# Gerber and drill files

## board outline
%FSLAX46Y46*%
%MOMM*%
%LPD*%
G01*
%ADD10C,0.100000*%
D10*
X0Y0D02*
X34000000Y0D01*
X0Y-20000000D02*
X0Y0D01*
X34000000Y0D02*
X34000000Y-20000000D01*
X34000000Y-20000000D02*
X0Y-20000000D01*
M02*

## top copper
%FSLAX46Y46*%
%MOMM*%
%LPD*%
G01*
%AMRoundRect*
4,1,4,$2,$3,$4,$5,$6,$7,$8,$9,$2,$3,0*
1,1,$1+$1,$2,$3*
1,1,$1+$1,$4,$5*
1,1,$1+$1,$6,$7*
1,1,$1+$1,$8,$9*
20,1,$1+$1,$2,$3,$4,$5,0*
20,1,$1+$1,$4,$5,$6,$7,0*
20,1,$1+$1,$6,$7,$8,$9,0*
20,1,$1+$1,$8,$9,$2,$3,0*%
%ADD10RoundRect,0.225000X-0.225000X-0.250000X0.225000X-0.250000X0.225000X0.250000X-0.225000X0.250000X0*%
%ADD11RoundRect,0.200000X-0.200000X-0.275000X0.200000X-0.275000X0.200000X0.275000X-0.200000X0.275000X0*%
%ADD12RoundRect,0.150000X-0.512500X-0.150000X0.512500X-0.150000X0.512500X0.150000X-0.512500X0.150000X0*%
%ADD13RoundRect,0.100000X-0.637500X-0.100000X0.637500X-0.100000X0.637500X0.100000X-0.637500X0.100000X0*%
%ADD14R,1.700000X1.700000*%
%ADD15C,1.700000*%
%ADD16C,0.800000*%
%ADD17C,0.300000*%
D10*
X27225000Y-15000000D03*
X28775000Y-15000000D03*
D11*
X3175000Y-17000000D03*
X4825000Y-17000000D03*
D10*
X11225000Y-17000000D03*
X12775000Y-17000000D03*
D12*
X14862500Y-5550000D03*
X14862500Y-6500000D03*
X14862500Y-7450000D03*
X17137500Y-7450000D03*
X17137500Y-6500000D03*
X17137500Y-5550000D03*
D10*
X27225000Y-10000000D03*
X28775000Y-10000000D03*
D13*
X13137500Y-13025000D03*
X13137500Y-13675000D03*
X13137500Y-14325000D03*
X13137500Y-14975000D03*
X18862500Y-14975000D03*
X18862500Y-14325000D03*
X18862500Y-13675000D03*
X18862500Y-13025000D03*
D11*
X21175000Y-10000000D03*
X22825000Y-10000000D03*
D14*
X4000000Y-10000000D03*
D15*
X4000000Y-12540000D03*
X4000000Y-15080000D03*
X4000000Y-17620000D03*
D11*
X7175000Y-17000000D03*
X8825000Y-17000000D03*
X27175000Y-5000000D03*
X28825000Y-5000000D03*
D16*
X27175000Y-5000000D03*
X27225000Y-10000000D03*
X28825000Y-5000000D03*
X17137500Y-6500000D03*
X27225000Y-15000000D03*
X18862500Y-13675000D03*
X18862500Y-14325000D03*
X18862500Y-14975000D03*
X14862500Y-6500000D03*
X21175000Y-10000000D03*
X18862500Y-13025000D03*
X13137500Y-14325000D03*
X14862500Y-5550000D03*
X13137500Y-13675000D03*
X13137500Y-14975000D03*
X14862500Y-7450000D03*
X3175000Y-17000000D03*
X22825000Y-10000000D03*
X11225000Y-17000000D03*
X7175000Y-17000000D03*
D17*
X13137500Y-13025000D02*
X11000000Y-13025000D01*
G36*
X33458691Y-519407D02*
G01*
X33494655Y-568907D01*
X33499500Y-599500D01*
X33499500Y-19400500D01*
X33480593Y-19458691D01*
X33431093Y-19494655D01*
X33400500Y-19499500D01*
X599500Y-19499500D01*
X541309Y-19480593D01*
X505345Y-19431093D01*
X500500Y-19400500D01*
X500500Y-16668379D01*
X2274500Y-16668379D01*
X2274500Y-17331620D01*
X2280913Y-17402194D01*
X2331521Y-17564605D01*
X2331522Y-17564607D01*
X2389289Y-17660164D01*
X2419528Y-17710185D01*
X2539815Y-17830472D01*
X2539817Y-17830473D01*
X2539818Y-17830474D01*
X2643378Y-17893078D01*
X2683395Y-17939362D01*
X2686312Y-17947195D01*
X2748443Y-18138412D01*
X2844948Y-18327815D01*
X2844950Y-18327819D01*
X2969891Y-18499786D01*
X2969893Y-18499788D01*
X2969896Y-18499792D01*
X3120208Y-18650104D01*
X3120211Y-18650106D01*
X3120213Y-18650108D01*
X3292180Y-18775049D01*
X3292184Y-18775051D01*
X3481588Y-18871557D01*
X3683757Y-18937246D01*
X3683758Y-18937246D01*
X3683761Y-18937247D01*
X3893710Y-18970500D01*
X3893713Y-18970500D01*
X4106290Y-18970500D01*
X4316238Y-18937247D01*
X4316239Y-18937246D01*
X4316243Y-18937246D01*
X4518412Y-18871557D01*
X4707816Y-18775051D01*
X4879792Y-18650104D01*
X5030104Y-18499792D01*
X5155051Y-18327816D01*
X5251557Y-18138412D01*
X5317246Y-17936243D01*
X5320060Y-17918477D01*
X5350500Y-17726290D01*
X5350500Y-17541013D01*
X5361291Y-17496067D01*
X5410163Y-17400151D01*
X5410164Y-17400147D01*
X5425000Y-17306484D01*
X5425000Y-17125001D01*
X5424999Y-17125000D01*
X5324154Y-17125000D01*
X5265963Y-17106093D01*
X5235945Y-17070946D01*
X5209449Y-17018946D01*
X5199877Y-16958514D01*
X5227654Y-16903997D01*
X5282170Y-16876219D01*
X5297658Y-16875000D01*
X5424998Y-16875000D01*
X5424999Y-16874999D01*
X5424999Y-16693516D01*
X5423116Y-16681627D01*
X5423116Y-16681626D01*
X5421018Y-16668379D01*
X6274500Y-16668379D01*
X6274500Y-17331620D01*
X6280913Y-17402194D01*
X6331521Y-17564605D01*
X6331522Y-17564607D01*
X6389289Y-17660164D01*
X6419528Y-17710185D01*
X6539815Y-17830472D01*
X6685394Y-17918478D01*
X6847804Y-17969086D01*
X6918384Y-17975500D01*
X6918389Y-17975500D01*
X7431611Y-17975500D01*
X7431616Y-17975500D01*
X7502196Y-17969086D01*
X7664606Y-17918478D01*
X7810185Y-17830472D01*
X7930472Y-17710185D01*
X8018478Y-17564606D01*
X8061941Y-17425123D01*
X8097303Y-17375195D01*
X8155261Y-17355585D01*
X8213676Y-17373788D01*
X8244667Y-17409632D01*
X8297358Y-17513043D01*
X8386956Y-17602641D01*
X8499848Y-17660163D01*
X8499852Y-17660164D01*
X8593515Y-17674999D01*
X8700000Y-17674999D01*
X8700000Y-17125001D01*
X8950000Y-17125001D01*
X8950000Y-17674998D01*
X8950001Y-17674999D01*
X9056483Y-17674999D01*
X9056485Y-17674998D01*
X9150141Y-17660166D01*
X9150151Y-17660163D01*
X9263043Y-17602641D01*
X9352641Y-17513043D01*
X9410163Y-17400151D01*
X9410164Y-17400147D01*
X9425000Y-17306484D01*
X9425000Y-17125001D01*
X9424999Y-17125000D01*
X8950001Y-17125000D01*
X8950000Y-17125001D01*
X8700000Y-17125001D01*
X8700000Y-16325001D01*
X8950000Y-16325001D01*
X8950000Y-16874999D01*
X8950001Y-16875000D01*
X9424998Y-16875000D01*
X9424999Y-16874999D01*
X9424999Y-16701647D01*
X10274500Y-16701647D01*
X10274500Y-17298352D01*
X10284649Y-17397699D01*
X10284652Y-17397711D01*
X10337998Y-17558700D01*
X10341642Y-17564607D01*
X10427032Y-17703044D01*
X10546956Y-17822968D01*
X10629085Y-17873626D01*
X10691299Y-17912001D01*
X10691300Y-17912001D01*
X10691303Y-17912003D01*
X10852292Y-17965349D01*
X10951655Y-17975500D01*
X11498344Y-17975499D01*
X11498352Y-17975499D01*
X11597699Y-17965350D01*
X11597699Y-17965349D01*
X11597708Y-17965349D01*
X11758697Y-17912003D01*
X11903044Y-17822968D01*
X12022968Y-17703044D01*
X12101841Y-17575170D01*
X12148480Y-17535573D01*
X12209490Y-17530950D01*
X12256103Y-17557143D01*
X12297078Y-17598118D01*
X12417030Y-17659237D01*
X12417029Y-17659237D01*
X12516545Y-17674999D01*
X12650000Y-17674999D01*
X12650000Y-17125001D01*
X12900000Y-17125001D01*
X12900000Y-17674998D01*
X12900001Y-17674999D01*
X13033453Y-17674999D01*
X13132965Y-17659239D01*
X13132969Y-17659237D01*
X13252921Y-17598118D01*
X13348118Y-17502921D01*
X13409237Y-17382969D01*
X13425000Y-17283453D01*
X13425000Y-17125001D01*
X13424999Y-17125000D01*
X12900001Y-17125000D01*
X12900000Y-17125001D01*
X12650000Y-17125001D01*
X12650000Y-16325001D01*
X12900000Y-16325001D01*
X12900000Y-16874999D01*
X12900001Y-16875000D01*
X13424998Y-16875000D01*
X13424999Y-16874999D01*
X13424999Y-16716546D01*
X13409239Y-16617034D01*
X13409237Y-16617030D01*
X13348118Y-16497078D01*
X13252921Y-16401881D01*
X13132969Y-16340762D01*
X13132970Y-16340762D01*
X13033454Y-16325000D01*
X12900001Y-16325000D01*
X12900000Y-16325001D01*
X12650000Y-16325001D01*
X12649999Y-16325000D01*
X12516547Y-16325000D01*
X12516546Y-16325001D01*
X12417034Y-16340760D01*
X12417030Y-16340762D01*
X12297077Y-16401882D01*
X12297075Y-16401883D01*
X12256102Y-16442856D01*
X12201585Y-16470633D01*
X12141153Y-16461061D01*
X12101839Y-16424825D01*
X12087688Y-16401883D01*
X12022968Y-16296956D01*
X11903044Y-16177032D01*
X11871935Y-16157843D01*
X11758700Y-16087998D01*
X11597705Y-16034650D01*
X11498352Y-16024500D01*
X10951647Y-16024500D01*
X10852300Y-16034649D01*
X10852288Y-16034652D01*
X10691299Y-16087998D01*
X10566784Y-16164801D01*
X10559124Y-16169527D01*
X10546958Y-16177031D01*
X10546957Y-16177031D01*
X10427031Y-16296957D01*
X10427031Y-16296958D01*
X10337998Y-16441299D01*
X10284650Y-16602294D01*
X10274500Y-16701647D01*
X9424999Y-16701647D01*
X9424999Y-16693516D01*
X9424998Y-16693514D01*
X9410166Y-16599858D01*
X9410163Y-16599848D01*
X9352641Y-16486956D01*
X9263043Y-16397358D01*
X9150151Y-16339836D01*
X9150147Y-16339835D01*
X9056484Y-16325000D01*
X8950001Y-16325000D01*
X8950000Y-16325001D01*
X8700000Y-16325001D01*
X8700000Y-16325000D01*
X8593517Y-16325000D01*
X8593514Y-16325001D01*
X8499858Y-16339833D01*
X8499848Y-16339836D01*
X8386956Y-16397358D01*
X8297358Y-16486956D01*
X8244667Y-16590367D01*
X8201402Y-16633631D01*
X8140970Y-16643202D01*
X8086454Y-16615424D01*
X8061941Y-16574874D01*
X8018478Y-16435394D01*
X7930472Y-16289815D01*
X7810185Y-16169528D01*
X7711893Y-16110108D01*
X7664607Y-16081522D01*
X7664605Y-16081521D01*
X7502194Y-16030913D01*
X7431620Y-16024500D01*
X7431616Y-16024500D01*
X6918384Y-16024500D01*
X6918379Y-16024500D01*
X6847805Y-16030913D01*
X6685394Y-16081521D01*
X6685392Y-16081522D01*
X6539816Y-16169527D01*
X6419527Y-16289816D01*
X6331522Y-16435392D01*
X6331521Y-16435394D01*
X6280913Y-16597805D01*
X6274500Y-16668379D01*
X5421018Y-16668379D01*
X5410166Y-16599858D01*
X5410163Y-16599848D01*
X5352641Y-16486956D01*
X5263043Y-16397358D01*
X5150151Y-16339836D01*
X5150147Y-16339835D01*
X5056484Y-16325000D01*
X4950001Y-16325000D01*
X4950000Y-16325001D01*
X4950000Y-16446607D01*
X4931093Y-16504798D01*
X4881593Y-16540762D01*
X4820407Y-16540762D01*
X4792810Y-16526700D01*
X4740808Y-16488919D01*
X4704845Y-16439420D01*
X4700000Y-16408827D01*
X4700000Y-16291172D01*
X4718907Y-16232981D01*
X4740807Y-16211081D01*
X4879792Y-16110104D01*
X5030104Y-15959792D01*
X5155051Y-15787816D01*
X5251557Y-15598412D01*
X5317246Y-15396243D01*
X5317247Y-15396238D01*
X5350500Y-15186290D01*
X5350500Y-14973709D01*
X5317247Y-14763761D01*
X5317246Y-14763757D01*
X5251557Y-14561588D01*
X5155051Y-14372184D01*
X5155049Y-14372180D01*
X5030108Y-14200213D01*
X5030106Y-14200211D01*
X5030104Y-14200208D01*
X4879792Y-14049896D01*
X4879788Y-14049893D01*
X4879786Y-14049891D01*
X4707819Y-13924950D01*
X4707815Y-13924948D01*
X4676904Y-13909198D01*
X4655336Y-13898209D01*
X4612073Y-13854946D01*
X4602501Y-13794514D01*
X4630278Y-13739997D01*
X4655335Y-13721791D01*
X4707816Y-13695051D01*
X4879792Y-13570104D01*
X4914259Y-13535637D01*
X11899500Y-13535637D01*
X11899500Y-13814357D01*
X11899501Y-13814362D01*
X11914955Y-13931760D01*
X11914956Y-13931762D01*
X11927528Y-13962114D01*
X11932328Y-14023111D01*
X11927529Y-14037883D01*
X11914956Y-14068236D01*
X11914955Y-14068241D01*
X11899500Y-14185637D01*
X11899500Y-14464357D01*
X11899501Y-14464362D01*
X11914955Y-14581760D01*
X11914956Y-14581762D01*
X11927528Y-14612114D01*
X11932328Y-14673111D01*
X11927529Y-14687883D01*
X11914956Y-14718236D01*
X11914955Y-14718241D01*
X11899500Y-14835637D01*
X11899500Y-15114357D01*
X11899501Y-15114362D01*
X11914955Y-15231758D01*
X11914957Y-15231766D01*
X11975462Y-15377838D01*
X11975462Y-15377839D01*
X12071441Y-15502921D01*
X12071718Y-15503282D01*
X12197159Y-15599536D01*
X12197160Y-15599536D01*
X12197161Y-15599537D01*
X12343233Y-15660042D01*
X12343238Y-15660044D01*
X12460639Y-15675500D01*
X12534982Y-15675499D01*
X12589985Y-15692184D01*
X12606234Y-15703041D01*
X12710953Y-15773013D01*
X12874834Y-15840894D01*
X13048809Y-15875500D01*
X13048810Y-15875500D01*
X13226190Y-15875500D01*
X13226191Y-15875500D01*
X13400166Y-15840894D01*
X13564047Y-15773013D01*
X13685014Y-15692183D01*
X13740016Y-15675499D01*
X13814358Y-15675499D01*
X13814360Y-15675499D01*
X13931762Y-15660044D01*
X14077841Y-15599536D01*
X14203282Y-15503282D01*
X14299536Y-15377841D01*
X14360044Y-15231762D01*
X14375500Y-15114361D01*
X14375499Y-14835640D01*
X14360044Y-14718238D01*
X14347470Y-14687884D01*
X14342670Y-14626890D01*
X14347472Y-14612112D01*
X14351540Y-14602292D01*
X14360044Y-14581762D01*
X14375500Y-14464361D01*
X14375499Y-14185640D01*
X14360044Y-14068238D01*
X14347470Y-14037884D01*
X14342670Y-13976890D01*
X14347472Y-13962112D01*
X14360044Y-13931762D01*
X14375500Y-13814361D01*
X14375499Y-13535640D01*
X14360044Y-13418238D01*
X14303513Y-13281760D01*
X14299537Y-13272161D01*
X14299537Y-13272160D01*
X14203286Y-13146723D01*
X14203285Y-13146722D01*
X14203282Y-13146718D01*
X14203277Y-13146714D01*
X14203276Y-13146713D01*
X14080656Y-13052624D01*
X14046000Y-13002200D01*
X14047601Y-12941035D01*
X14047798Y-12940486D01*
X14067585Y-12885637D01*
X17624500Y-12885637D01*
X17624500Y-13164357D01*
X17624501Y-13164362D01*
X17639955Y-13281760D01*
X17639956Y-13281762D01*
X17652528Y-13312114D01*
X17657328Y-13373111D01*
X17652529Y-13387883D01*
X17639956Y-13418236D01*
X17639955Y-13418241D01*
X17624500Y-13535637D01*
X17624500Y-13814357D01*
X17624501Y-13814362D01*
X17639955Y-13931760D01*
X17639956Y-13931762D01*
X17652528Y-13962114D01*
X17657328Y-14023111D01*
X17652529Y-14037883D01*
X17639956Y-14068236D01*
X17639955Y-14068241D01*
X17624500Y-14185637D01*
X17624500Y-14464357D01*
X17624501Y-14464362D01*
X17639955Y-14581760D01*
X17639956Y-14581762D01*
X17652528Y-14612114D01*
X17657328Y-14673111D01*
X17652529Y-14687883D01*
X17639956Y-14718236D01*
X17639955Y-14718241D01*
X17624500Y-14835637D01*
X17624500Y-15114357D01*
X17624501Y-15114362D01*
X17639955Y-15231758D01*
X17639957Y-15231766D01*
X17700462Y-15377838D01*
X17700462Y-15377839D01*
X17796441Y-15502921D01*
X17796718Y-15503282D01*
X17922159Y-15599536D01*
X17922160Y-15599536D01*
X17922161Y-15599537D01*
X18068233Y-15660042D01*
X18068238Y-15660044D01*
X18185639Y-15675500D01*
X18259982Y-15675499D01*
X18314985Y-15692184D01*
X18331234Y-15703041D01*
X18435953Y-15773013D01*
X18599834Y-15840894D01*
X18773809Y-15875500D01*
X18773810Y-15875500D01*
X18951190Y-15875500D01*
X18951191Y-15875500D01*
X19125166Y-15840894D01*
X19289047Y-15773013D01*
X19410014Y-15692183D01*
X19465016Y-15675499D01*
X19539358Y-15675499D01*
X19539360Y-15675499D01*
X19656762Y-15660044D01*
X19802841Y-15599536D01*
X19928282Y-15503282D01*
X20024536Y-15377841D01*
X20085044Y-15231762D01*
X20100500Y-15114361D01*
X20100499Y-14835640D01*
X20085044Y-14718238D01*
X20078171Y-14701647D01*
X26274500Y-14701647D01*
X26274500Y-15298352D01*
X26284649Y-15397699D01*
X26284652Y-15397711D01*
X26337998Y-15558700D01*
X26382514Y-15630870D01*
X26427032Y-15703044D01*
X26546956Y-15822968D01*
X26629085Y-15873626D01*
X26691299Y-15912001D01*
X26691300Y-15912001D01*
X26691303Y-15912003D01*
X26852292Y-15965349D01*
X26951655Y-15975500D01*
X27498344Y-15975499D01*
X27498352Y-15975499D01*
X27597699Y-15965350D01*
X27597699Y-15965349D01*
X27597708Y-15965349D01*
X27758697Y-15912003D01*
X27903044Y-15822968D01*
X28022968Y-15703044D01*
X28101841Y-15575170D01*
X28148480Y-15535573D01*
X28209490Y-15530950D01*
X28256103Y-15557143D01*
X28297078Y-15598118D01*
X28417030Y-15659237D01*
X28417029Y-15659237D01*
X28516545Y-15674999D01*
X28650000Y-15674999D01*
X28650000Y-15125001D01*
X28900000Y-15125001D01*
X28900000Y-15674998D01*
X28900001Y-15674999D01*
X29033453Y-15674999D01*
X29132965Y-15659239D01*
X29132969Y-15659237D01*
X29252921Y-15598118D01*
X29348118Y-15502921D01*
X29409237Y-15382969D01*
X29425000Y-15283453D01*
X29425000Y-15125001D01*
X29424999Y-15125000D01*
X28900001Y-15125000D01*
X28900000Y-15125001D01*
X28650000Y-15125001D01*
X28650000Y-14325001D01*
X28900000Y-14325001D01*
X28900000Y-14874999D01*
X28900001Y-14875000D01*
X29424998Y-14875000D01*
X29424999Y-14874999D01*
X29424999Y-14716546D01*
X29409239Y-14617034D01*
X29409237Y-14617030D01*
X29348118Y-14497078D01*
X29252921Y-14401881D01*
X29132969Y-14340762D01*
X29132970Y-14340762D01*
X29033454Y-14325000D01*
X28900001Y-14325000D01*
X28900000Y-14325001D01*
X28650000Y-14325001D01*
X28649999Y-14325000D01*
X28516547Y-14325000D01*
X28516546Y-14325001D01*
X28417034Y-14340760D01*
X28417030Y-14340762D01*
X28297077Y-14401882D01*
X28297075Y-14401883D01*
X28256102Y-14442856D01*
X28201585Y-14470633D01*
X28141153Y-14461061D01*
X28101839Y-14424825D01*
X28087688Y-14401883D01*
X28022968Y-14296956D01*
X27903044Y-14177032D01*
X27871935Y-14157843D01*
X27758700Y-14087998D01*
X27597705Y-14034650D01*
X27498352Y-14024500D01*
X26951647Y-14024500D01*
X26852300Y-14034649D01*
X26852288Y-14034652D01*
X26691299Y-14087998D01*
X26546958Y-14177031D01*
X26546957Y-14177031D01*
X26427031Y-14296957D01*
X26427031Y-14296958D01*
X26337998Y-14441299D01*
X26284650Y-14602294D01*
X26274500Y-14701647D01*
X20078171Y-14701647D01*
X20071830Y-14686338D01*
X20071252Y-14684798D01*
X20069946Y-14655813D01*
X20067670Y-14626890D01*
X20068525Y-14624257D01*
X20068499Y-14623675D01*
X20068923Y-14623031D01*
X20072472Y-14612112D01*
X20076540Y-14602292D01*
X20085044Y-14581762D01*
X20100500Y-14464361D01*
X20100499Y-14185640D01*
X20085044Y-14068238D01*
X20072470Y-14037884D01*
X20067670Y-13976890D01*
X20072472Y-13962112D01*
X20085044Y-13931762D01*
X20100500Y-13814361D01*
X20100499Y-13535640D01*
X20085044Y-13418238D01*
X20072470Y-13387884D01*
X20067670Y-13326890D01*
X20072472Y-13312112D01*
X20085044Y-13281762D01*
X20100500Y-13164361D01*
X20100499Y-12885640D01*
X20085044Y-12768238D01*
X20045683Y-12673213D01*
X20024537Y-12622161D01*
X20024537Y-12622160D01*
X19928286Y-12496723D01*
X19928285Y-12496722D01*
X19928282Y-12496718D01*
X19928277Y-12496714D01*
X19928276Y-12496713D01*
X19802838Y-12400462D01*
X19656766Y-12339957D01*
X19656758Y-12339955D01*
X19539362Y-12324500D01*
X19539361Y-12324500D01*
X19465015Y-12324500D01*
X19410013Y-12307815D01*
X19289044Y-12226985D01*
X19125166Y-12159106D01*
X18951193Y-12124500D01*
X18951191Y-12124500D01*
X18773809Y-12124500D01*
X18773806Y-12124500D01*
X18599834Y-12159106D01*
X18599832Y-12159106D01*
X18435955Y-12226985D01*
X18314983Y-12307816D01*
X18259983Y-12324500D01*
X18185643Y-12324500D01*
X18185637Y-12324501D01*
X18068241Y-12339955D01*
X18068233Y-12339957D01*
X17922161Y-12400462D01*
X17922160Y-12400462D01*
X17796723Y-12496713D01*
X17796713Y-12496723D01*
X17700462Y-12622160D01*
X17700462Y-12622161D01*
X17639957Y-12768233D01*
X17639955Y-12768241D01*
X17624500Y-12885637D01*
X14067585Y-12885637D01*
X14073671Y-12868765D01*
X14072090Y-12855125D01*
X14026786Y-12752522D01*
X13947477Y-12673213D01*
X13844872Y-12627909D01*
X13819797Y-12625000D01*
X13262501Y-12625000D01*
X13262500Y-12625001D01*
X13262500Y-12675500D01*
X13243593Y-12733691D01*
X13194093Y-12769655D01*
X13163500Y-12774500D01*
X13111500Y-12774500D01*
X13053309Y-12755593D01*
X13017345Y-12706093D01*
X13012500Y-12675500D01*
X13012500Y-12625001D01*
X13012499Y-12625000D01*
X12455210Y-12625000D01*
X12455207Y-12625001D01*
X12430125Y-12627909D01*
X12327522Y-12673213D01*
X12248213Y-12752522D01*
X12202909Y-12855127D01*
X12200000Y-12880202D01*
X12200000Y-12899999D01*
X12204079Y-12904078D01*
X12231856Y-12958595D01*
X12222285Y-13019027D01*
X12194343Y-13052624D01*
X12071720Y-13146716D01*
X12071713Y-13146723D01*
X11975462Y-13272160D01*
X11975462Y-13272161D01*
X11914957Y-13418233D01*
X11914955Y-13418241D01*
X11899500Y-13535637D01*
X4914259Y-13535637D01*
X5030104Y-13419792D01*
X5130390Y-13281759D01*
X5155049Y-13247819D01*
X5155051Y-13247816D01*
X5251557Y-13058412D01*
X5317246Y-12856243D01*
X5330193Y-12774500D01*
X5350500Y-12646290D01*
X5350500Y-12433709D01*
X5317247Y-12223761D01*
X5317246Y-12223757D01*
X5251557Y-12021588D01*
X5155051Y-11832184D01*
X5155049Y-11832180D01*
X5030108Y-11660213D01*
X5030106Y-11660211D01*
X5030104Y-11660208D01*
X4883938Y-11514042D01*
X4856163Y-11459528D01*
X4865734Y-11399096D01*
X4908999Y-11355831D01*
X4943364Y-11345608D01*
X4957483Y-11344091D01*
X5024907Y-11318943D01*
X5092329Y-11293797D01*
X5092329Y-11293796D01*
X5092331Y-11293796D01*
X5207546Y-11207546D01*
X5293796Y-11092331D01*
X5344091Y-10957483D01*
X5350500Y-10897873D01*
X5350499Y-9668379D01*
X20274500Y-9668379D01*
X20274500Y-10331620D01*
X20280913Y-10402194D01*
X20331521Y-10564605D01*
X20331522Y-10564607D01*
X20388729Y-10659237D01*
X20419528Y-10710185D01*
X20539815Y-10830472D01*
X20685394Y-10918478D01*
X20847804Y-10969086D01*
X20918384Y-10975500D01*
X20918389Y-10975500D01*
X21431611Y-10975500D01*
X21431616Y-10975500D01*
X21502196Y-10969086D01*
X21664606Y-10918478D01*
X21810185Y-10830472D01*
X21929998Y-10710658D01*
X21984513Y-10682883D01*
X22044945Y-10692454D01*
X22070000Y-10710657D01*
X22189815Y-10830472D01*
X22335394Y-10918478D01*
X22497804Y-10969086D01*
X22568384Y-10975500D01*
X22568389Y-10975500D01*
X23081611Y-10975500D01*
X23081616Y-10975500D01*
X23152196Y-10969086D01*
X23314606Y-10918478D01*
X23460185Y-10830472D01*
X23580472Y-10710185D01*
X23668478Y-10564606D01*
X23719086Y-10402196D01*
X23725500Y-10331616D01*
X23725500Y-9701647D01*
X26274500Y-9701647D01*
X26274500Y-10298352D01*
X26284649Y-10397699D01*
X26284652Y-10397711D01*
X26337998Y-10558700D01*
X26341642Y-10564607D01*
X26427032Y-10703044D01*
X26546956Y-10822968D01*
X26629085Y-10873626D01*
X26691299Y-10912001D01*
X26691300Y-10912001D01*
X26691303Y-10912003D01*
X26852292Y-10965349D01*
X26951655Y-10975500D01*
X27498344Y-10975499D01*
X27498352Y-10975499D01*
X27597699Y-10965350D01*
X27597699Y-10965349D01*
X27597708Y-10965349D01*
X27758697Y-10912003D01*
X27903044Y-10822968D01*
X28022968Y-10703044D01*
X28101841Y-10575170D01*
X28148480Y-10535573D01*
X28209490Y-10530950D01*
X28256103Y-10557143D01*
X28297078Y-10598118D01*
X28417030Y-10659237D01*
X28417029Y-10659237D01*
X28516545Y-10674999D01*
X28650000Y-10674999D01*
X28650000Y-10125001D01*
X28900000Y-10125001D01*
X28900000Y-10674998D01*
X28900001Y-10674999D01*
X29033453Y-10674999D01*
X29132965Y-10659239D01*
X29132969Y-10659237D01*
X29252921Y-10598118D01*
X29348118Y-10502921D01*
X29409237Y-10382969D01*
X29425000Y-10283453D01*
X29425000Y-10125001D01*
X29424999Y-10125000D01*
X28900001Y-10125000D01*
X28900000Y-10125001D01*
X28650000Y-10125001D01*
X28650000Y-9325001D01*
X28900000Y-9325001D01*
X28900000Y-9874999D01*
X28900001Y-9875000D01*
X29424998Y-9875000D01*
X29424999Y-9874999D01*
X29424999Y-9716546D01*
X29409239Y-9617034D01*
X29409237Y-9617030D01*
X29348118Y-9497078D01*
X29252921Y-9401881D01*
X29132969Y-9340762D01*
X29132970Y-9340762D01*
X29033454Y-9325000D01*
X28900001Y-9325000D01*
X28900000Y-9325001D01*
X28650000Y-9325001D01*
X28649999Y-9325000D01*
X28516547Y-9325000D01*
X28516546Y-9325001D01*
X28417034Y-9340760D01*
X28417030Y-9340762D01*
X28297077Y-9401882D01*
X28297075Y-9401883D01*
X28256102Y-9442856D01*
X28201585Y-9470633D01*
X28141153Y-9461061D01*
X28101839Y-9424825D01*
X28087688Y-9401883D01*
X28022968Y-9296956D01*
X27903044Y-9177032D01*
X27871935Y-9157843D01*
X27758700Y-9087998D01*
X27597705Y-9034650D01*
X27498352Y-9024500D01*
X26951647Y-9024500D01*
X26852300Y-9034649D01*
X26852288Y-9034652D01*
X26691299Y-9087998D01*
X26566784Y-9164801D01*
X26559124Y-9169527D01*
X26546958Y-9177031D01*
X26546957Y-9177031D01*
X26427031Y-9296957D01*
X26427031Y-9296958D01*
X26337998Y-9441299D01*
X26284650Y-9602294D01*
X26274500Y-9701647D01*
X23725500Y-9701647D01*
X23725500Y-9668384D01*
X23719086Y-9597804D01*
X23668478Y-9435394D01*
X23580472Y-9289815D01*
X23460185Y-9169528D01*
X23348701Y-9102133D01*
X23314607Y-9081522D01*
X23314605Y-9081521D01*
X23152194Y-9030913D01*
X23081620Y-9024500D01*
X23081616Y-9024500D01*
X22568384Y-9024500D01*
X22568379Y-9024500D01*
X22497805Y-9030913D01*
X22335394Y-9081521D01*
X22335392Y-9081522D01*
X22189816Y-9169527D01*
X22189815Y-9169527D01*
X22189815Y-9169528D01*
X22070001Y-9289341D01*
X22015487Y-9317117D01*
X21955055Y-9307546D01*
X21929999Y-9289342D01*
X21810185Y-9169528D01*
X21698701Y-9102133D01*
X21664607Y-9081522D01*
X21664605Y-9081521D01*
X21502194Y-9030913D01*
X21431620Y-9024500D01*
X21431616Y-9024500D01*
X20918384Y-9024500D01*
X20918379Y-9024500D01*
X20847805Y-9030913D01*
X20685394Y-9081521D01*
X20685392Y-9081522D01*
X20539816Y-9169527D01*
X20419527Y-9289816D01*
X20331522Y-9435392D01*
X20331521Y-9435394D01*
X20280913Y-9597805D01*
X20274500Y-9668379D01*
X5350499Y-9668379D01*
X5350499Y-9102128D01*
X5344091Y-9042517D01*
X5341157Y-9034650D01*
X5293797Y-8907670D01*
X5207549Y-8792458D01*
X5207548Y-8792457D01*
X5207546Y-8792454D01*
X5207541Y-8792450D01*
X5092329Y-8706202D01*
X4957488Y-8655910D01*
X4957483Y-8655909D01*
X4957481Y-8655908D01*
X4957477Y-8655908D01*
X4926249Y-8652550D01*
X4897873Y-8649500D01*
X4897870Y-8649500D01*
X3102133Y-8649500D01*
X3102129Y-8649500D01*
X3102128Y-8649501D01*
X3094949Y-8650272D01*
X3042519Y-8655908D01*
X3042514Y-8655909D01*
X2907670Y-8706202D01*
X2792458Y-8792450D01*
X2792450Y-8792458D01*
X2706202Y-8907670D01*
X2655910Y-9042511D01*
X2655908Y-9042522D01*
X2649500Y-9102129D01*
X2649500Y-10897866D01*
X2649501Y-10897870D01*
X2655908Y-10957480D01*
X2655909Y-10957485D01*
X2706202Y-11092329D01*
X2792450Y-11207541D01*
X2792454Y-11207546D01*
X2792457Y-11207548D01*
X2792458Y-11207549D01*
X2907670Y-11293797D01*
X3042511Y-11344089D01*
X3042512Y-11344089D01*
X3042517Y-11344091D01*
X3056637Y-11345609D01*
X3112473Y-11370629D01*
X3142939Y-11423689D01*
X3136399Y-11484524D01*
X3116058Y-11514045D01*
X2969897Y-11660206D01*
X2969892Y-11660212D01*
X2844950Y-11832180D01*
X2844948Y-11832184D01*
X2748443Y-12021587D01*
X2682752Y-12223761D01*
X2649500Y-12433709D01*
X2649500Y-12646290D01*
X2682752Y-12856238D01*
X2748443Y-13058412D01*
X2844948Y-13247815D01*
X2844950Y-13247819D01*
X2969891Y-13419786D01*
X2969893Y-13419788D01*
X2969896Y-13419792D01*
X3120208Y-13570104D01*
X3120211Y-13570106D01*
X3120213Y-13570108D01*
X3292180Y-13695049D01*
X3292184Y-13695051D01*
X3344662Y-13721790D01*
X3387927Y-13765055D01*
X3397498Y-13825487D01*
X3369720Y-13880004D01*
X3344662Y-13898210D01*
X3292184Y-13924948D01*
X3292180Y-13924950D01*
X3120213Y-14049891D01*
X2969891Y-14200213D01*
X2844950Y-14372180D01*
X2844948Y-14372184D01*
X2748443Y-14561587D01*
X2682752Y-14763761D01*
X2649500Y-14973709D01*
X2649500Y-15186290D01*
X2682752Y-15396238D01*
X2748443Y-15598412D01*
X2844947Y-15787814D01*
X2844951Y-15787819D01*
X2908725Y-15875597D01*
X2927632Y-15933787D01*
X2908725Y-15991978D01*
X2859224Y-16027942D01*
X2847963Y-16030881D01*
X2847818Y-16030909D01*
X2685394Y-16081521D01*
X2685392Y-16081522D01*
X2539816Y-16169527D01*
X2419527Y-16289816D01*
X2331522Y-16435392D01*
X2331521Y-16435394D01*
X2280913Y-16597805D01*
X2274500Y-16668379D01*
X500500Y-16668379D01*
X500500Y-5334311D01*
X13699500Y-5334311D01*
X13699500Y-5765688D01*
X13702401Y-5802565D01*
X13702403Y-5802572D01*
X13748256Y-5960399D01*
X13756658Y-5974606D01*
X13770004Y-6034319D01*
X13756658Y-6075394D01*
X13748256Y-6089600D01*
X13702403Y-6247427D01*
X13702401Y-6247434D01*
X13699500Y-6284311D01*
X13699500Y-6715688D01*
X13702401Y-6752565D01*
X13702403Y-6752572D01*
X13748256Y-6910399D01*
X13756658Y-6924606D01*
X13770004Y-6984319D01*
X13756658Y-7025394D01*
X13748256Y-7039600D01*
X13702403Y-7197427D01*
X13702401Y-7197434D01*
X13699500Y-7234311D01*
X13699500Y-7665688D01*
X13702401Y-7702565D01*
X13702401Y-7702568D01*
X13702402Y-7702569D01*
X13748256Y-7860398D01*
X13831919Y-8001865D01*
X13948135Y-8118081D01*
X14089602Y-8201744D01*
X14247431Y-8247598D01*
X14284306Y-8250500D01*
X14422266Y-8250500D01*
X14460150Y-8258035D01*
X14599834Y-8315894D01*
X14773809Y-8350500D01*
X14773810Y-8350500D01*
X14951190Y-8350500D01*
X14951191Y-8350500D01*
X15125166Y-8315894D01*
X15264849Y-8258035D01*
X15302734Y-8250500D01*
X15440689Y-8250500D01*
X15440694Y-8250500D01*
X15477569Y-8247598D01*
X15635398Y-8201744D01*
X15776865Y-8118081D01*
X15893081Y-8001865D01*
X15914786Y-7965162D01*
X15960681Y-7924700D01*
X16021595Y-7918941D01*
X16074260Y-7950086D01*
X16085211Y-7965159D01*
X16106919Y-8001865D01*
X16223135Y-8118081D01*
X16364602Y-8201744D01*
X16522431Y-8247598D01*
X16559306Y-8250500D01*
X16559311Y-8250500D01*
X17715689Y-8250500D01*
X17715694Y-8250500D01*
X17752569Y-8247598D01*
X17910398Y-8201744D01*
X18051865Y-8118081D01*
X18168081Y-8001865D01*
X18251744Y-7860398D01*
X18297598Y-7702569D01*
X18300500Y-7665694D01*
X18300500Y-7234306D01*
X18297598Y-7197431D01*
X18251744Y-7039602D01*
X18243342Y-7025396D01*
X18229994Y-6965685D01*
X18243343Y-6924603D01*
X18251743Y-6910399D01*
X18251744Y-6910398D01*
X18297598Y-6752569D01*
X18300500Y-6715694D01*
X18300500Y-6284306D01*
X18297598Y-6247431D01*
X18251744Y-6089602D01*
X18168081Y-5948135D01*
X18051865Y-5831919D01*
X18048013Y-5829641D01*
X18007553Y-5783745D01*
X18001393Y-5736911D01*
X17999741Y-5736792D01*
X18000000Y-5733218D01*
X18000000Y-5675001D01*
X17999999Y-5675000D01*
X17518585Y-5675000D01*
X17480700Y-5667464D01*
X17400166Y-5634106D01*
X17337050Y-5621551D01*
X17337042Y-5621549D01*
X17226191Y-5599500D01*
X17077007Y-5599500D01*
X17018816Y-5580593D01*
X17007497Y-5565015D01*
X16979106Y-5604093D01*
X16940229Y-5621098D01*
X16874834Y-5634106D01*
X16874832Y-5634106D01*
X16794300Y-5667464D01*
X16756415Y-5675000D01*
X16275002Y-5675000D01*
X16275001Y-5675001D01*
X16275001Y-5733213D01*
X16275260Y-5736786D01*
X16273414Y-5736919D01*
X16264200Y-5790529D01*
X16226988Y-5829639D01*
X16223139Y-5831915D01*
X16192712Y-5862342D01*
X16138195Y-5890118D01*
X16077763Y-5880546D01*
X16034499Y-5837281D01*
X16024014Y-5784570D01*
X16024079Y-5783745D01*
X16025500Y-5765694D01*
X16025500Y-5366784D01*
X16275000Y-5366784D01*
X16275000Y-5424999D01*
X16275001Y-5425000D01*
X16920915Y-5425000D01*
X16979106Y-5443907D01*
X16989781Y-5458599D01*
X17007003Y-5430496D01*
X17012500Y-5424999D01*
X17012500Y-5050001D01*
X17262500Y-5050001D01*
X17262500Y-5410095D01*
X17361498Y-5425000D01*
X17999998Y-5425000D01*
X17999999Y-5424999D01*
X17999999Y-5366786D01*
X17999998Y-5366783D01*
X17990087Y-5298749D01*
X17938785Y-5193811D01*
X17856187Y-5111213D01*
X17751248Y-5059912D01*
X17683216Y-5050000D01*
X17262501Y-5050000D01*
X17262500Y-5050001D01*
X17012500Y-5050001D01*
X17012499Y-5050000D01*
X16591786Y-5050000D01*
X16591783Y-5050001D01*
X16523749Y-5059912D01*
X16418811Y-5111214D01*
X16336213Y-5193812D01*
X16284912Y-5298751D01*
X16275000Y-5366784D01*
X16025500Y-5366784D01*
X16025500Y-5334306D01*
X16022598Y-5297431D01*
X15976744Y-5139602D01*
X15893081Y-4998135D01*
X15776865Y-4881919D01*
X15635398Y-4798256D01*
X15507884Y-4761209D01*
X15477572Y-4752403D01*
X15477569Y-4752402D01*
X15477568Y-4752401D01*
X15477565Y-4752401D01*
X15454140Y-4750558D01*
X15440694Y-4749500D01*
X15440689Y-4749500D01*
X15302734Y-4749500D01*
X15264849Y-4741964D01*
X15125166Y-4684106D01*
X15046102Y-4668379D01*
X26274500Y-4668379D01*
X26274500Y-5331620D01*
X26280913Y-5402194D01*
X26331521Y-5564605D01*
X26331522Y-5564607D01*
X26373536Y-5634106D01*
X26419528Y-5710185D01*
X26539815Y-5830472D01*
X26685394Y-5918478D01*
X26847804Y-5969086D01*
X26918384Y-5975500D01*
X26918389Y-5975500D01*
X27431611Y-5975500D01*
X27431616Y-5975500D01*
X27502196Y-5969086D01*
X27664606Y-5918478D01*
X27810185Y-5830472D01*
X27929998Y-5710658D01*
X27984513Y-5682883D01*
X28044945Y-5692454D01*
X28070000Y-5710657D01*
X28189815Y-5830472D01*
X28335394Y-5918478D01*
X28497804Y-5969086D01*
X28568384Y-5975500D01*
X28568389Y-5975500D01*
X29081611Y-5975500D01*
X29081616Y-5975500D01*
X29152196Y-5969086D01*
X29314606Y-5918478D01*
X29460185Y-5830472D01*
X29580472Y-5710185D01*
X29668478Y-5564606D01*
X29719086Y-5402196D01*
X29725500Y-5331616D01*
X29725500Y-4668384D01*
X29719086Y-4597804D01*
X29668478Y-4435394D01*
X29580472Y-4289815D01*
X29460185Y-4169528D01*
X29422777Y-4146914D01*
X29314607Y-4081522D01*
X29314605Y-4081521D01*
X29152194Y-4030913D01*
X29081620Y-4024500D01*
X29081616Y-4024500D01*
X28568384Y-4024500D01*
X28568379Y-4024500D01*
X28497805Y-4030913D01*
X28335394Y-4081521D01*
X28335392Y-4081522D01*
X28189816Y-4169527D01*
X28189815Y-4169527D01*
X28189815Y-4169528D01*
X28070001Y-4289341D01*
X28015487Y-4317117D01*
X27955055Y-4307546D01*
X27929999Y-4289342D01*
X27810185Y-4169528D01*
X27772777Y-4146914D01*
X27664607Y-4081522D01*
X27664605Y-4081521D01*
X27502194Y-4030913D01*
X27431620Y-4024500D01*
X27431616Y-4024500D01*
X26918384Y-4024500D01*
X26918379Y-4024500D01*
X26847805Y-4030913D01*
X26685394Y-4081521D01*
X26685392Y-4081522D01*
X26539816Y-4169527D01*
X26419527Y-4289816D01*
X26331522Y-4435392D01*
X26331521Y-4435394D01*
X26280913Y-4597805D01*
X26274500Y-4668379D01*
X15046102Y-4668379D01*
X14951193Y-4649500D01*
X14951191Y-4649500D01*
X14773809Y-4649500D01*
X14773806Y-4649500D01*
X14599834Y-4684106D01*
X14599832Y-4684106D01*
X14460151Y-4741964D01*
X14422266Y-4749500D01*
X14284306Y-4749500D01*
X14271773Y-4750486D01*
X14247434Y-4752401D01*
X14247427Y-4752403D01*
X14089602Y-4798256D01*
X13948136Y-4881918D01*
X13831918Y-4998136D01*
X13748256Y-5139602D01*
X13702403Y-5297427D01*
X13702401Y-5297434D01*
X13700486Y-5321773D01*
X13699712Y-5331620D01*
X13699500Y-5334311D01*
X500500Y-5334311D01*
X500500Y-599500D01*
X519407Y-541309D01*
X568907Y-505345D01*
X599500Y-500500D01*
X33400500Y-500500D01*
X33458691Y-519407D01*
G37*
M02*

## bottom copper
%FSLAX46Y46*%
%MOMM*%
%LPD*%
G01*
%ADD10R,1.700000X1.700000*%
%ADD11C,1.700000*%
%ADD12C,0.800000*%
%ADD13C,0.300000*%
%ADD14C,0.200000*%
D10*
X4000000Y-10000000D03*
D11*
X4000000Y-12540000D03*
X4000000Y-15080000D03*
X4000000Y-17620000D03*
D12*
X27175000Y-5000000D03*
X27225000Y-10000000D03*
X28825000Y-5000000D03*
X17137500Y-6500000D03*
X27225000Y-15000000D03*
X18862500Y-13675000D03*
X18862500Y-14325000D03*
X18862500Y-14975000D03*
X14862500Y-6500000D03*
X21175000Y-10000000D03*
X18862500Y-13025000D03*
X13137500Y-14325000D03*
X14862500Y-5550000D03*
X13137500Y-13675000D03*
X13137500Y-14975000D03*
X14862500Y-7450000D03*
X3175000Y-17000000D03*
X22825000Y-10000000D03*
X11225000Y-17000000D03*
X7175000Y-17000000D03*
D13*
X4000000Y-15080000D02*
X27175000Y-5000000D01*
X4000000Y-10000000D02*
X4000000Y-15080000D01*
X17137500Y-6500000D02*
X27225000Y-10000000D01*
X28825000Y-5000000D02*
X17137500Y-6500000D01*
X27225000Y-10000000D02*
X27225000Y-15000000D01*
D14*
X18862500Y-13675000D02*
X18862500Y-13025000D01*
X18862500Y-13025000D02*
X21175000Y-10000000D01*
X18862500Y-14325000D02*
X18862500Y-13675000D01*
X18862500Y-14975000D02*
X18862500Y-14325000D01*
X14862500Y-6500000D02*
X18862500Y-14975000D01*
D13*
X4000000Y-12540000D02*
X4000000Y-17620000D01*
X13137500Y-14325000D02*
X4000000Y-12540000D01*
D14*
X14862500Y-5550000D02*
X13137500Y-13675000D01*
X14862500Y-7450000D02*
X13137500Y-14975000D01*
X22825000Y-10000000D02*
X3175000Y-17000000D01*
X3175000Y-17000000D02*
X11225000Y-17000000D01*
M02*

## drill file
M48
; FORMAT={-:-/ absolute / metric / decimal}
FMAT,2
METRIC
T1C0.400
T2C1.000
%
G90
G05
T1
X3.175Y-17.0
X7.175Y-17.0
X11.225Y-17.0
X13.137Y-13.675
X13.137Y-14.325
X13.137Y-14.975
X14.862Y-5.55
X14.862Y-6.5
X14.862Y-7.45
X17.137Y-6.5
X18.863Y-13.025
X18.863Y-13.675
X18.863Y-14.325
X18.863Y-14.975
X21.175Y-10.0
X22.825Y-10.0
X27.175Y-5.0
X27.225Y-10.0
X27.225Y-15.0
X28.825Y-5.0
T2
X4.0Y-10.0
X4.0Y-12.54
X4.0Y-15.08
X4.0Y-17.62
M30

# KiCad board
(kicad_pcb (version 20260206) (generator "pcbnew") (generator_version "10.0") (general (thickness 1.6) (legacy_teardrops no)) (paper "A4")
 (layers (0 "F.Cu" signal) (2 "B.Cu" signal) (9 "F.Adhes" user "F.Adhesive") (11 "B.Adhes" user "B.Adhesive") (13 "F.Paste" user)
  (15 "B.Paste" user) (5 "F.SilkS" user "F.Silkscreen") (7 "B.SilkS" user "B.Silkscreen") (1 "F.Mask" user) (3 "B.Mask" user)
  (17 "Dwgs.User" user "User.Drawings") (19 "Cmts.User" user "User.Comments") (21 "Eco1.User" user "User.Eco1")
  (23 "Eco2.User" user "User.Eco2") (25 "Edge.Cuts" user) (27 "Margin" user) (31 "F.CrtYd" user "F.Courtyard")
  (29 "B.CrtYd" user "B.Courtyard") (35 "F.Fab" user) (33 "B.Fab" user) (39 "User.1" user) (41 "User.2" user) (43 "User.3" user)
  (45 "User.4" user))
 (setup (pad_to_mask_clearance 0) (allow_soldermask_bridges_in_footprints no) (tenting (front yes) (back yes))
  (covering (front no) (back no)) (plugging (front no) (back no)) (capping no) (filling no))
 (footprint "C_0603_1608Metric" (layer "F.Cu") (at 28 15)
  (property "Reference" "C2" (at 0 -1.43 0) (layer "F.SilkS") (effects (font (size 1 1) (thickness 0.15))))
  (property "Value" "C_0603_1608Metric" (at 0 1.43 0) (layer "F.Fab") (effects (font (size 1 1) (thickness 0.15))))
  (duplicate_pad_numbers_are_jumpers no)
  (pad "1" smd roundrect (at -0.775 0) (size 0.9 0.95) (layers "F.Cu" "F.Mask" "F.Paste") (roundrect_rratio 0.25) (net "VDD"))
  (pad "2" smd roundrect (at 0.775 0) (size 0.9 0.95) (layers "F.Cu" "F.Mask" "F.Paste") (roundrect_rratio 0.25) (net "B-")))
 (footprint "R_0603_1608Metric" (layer "F.Cu") (at 4 17)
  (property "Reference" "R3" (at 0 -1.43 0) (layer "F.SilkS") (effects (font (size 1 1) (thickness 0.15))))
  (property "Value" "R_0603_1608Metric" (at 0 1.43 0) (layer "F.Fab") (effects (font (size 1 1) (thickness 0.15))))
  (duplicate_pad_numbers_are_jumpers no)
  (pad "1" smd roundrect (at -0.825 0) (size 0.8 0.95) (layers "F.Cu" "F.Mask" "F.Paste") (roundrect_rratio 0.25) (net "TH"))
  (pad "2" smd roundrect (at 0.825 0) (size 0.8 0.95) (layers "F.Cu" "F.Mask" "F.Paste") (roundrect_rratio 0.25) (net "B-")))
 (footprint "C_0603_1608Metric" (layer "F.Cu") (at 12 17)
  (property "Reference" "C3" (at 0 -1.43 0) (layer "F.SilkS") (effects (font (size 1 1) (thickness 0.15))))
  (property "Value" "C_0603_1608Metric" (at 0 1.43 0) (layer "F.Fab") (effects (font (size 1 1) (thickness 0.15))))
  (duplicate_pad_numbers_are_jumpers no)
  (pad "1" smd roundrect (at -0.775 0) (size 0.9 0.95) (layers "F.Cu" "F.Mask" "F.Paste") (roundrect_rratio 0.25) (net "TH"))
  (pad "2" smd roundrect (at 0.775 0) (size 0.9 0.95) (layers "F.Cu" "F.Mask" "F.Paste") (roundrect_rratio 0.25) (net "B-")))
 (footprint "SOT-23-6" (layer "F.Cu") (at 16 6.5)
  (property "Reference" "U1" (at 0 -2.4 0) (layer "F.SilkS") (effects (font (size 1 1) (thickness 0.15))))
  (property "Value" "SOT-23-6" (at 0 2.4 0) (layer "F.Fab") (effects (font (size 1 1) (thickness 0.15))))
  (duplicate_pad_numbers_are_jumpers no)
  (pad "1" smd roundrect (at -1.1375 -0.95) (size 1.325 0.6) (layers "F.Cu" "F.Mask" "F.Paste") (roundrect_rratio 0.25) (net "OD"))
  (pad "2" smd roundrect (at -1.1375 0) (size 1.325 0.6) (layers "F.Cu" "F.Mask" "F.Paste") (roundrect_rratio 0.25) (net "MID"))
  (pad "3" smd roundrect (at -1.1375 0.95) (size 1.325 0.6) (layers "F.Cu" "F.Mask" "F.Paste") (roundrect_rratio 0.25) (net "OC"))
  (pad "4" smd roundrect (at 1.1375 0.95) (size 1.325 0.6) (layers "F.Cu" "F.Mask" "F.Paste") (roundrect_rratio 0.25))
  (pad "5" smd roundrect (at 1.1375 0) (size 1.325 0.6) (layers "F.Cu" "F.Mask" "F.Paste") (roundrect_rratio 0.25) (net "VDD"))
  (pad "6" smd roundrect (at 1.1375 -0.95) (size 1.325 0.6) (layers "F.Cu" "F.Mask" "F.Paste") (roundrect_rratio 0.25) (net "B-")))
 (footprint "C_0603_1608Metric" (layer "F.Cu") (at 28 10)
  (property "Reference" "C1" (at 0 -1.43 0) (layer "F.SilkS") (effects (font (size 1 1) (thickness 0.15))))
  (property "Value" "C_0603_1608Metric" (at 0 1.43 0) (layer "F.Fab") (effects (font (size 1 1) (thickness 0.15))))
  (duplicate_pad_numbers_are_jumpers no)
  (pad "1" smd roundrect (at -0.775 0) (size 0.9 0.95) (layers "F.Cu" "F.Mask" "F.Paste") (roundrect_rratio 0.25) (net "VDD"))
  (pad "2" smd roundrect (at 0.775 0) (size 0.9 0.95) (layers "F.Cu" "F.Mask" "F.Paste") (roundrect_rratio 0.25) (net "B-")))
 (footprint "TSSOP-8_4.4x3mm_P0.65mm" (layer "F.Cu") (at 16 14)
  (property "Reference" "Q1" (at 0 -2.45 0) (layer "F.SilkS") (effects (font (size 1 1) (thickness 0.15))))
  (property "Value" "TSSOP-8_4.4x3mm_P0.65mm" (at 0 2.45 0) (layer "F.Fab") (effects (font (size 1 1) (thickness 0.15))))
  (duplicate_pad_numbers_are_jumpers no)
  (pad "1" smd roundrect (at -2.8625 -0.975) (size 1.475 0.4) (layers "F.Cu" "F.Mask" "F.Paste") (roundrect_rratio 0.25) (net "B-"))
  (pad "2" smd roundrect (at -2.8625 -0.325) (size 1.475 0.4) (layers "F.Cu" "F.Mask" "F.Paste") (roundrect_rratio 0.25) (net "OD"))
  (pad "3" smd roundrect (at -2.8625 0.325) (size 1.475 0.4) (layers "F.Cu" "F.Mask" "F.Paste") (roundrect_rratio 0.25) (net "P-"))
  (pad "4" smd roundrect (at -2.8625 0.975) (size 1.475 0.4) (layers "F.Cu" "F.Mask" "F.Paste") (roundrect_rratio 0.25) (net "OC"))
  (pad "5" smd roundrect (at 2.8625 0.975) (size 1.475 0.4) (layers "F.Cu" "F.Mask" "F.Paste") (roundrect_rratio 0.25) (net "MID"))
  (pad "6" smd roundrect (at 2.8625 0.325) (size 1.475 0.4) (layers "F.Cu" "F.Mask" "F.Paste") (roundrect_rratio 0.25) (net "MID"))
  (pad "7" smd roundrect (at 2.8625 -0.325) (size 1.475 0.4) (layers "F.Cu" "F.Mask" "F.Paste") (roundrect_rratio 0.25) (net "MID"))
  (pad "8" smd roundrect (at 2.8625 -0.975) (size 1.475 0.4) (layers "F.Cu" "F.Mask" "F.Paste") (roundrect_rratio 0.25) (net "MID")))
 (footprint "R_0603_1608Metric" (layer "F.Cu") (at 22 10)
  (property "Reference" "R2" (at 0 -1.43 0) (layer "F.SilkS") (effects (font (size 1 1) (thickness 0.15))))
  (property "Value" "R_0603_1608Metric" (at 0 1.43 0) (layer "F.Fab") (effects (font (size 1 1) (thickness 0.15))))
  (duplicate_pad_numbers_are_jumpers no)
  (pad "1" smd roundrect (at -0.825 0) (size 0.8 0.95) (layers "F.Cu" "F.Mask" "F.Paste") (roundrect_rratio 0.25) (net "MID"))
  (pad "2" smd roundrect (at 0.825 0) (size 0.8 0.95) (layers "F.Cu" "F.Mask" "F.Paste") (roundrect_rratio 0.25) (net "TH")))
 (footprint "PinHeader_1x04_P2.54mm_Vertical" (layer "F.Cu") (at 4 10)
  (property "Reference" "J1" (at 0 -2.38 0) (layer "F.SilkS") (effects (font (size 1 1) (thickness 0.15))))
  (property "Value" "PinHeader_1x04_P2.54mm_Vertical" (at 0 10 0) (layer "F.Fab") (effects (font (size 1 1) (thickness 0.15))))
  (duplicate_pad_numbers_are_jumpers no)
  (pad "1" thru_hole rect (at 0 0) (size 1.7 1.7) (drill 1) (layers "*.Cu" "*.Mask") (remove_unused_layers no) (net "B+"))
  (pad "2" thru_hole circle (at 0 2.54) (size 1.7 1.7) (drill 1) (layers "*.Cu" "*.Mask") (remove_unused_layers no) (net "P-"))
  (pad "3" thru_hole circle (at 0 5.08) (size 1.7 1.7) (drill 1) (layers "*.Cu" "*.Mask") (remove_unused_layers no) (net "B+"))
  (pad "4" thru_hole circle (at 0 7.62) (size 1.7 1.7) (drill 1) (layers "*.Cu" "*.Mask") (remove_unused_layers no) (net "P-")))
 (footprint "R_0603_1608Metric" (layer "F.Cu") (at 8 17)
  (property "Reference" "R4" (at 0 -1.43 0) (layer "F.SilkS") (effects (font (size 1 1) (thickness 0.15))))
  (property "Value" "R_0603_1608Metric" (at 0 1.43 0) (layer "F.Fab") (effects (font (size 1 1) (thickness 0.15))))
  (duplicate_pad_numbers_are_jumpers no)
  (pad "1" smd roundrect (at -0.825 0) (size 0.8 0.95) (layers "F.Cu" "F.Mask" "F.Paste") (roundrect_rratio 0.25) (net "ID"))
  (pad "2" smd roundrect (at 0.825 0) (size 0.8 0.95) (layers "F.Cu" "F.Mask" "F.Paste") (roundrect_rratio 0.25) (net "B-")))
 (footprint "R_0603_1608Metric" (layer "F.Cu") (at 28 5)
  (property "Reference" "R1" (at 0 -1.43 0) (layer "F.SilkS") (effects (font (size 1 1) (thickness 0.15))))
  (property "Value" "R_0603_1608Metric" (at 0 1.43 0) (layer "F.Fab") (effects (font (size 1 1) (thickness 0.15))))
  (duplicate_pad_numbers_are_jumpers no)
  (pad "1" smd roundrect (at -0.825 0) (size 0.8 0.95) (layers "F.Cu" "F.Mask" "F.Paste") (roundrect_rratio 0.25) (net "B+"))
  (pad "2" smd roundrect (at 0.825 0) (size 0.8 0.95) (layers "F.Cu" "F.Mask" "F.Paste") (roundrect_rratio 0.25) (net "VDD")))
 (gr_line (start 0 0) (end 34 0) (stroke (width 0.1) (type default)) (layer "Edge.Cuts"))
 (gr_line (start 0 20) (end 0 0) (stroke (width 0.1) (type default)) (layer "Edge.Cuts"))
 (gr_line (start 34 0) (end 34 20) (stroke (width 0.1) (type default)) (layer "Edge.Cuts"))
 (gr_line (start 34 20) (end 0 20) (stroke (width 0.1) (type default)) (layer "Edge.Cuts"))
 (via (at 27.175 5) (size 0.8) (drill 0.4) (layers "F.Cu" "B.Cu") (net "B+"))
 (segment (start 4 15.08) (end 27.175 5) (width 0.3) (layer "B.Cu") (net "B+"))
 (segment (start 4 10) (end 4 15.08) (width 0.3) (layer "B.Cu") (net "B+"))
 (via (at 27.225 10) (size 0.8) (drill 0.4) (layers "F.Cu" "B.Cu") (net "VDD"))
 (via (at 28.825 5) (size 0.8) (drill 0.4) (layers "F.Cu" "B.Cu") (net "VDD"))
 (via (at 17.1375 6.5) (size 0.8) (drill 0.4) (layers "F.Cu" "B.Cu") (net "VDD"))
 (via (at 27.225 15) (size 0.8) (drill 0.4) (layers "F.Cu" "B.Cu") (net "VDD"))
 (segment (start 17.1375 6.5) (end 27.225 10) (width 0.3) (layer "B.Cu") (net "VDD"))
 (segment (start 28.825 5) (end 17.1375 6.5) (width 0.3) (layer "B.Cu") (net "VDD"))
 (segment (start 27.225 10) (end 27.225 15) (width 0.3) (layer "B.Cu") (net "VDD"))
 (segment (start 13.1375 13.025) (end 11 13.025) (width 0.3) (layer "F.Cu") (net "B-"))
 (via (at 18.8625 13.675) (size 0.8) (drill 0.4) (layers "F.Cu" "B.Cu") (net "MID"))
 (via (at 18.8625 14.325) (size 0.8) (drill 0.4) (layers "F.Cu" "B.Cu") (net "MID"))
 (via (at 18.8625 14.975) (size 0.8) (drill 0.4) (layers "F.Cu" "B.Cu") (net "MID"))
 (via (at 14.8625 6.5) (size 0.8) (drill 0.4) (layers "F.Cu" "B.Cu") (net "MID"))
 (via (at 21.175 10) (size 0.8) (drill 0.4) (layers "F.Cu" "B.Cu") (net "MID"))
 (via (at 18.8625 13.025) (size 0.8) (drill 0.4) (layers "F.Cu" "B.Cu") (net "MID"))
 (segment (start 18.8625 13.675) (end 18.8625 13.025) (width 0.2) (layer "B.Cu") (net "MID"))
 (segment (start 18.8625 13.025) (end 21.175 10) (width 0.2) (layer "B.Cu") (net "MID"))
 (segment (start 18.8625 14.325) (end 18.8625 13.675) (width 0.2) (layer "B.Cu") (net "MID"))
 (segment (start 18.8625 14.975) (end 18.8625 14.325) (width 0.2) (layer "B.Cu") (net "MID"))
 (segment (start 14.8625 6.5) (end 18.8625 14.975) (width 0.2) (layer "B.Cu") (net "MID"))
 (via (at 13.1375 14.325) (size 0.8) (drill 0.4) (layers "F.Cu" "B.Cu") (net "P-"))
 (segment (start 4 12.54) (end 4 17.62) (width 0.3) (layer "B.Cu") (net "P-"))
 (segment (start 13.1375 14.325) (end 4 12.54) (width 0.3) (layer "B.Cu") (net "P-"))
 (via (at 14.8625 5.55) (size 0.8) (drill 0.4) (layers "F.Cu" "B.Cu") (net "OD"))
 (via (at 13.1375 13.675) (size 0.8) (drill 0.4) (layers "F.Cu" "B.Cu") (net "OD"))
 (segment (start 14.8625 5.55) (end 13.1375 13.675) (width 0.2) (layer "B.Cu") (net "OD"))
 (via (at 13.1375 14.975) (size 0.8) (drill 0.4) (layers "F.Cu" "B.Cu") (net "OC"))
 (via (at 14.8625 7.45) (size 0.8) (drill 0.4) (layers "F.Cu" "B.Cu") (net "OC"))
 (segment (start 14.8625 7.45) (end 13.1375 14.975) (width 0.2) (layer "B.Cu") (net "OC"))
 (via (at 3.175 17) (size 0.8) (drill 0.4) (layers "F.Cu" "B.Cu") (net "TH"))
 (via (at 22.825 10) (size 0.8) (drill 0.4) (layers "F.Cu" "B.Cu") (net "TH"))
 (via (at 11.225 17) (size 0.8) (drill 0.4) (layers "F.Cu" "B.Cu") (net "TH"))
 (segment (start 22.825 10) (end 3.175 17) (width 0.2) (layer "B.Cu") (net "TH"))
 (segment (start 3.175 17) (end 11.225 17) (width 0.2) (layer "B.Cu") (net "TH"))
 (via (at 7.175 17) (size 0.8) (drill 0.4) (layers "F.Cu" "B.Cu") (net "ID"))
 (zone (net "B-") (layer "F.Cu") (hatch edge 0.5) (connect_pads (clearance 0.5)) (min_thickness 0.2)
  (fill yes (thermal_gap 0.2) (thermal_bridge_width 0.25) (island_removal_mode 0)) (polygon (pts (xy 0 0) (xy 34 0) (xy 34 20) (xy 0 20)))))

